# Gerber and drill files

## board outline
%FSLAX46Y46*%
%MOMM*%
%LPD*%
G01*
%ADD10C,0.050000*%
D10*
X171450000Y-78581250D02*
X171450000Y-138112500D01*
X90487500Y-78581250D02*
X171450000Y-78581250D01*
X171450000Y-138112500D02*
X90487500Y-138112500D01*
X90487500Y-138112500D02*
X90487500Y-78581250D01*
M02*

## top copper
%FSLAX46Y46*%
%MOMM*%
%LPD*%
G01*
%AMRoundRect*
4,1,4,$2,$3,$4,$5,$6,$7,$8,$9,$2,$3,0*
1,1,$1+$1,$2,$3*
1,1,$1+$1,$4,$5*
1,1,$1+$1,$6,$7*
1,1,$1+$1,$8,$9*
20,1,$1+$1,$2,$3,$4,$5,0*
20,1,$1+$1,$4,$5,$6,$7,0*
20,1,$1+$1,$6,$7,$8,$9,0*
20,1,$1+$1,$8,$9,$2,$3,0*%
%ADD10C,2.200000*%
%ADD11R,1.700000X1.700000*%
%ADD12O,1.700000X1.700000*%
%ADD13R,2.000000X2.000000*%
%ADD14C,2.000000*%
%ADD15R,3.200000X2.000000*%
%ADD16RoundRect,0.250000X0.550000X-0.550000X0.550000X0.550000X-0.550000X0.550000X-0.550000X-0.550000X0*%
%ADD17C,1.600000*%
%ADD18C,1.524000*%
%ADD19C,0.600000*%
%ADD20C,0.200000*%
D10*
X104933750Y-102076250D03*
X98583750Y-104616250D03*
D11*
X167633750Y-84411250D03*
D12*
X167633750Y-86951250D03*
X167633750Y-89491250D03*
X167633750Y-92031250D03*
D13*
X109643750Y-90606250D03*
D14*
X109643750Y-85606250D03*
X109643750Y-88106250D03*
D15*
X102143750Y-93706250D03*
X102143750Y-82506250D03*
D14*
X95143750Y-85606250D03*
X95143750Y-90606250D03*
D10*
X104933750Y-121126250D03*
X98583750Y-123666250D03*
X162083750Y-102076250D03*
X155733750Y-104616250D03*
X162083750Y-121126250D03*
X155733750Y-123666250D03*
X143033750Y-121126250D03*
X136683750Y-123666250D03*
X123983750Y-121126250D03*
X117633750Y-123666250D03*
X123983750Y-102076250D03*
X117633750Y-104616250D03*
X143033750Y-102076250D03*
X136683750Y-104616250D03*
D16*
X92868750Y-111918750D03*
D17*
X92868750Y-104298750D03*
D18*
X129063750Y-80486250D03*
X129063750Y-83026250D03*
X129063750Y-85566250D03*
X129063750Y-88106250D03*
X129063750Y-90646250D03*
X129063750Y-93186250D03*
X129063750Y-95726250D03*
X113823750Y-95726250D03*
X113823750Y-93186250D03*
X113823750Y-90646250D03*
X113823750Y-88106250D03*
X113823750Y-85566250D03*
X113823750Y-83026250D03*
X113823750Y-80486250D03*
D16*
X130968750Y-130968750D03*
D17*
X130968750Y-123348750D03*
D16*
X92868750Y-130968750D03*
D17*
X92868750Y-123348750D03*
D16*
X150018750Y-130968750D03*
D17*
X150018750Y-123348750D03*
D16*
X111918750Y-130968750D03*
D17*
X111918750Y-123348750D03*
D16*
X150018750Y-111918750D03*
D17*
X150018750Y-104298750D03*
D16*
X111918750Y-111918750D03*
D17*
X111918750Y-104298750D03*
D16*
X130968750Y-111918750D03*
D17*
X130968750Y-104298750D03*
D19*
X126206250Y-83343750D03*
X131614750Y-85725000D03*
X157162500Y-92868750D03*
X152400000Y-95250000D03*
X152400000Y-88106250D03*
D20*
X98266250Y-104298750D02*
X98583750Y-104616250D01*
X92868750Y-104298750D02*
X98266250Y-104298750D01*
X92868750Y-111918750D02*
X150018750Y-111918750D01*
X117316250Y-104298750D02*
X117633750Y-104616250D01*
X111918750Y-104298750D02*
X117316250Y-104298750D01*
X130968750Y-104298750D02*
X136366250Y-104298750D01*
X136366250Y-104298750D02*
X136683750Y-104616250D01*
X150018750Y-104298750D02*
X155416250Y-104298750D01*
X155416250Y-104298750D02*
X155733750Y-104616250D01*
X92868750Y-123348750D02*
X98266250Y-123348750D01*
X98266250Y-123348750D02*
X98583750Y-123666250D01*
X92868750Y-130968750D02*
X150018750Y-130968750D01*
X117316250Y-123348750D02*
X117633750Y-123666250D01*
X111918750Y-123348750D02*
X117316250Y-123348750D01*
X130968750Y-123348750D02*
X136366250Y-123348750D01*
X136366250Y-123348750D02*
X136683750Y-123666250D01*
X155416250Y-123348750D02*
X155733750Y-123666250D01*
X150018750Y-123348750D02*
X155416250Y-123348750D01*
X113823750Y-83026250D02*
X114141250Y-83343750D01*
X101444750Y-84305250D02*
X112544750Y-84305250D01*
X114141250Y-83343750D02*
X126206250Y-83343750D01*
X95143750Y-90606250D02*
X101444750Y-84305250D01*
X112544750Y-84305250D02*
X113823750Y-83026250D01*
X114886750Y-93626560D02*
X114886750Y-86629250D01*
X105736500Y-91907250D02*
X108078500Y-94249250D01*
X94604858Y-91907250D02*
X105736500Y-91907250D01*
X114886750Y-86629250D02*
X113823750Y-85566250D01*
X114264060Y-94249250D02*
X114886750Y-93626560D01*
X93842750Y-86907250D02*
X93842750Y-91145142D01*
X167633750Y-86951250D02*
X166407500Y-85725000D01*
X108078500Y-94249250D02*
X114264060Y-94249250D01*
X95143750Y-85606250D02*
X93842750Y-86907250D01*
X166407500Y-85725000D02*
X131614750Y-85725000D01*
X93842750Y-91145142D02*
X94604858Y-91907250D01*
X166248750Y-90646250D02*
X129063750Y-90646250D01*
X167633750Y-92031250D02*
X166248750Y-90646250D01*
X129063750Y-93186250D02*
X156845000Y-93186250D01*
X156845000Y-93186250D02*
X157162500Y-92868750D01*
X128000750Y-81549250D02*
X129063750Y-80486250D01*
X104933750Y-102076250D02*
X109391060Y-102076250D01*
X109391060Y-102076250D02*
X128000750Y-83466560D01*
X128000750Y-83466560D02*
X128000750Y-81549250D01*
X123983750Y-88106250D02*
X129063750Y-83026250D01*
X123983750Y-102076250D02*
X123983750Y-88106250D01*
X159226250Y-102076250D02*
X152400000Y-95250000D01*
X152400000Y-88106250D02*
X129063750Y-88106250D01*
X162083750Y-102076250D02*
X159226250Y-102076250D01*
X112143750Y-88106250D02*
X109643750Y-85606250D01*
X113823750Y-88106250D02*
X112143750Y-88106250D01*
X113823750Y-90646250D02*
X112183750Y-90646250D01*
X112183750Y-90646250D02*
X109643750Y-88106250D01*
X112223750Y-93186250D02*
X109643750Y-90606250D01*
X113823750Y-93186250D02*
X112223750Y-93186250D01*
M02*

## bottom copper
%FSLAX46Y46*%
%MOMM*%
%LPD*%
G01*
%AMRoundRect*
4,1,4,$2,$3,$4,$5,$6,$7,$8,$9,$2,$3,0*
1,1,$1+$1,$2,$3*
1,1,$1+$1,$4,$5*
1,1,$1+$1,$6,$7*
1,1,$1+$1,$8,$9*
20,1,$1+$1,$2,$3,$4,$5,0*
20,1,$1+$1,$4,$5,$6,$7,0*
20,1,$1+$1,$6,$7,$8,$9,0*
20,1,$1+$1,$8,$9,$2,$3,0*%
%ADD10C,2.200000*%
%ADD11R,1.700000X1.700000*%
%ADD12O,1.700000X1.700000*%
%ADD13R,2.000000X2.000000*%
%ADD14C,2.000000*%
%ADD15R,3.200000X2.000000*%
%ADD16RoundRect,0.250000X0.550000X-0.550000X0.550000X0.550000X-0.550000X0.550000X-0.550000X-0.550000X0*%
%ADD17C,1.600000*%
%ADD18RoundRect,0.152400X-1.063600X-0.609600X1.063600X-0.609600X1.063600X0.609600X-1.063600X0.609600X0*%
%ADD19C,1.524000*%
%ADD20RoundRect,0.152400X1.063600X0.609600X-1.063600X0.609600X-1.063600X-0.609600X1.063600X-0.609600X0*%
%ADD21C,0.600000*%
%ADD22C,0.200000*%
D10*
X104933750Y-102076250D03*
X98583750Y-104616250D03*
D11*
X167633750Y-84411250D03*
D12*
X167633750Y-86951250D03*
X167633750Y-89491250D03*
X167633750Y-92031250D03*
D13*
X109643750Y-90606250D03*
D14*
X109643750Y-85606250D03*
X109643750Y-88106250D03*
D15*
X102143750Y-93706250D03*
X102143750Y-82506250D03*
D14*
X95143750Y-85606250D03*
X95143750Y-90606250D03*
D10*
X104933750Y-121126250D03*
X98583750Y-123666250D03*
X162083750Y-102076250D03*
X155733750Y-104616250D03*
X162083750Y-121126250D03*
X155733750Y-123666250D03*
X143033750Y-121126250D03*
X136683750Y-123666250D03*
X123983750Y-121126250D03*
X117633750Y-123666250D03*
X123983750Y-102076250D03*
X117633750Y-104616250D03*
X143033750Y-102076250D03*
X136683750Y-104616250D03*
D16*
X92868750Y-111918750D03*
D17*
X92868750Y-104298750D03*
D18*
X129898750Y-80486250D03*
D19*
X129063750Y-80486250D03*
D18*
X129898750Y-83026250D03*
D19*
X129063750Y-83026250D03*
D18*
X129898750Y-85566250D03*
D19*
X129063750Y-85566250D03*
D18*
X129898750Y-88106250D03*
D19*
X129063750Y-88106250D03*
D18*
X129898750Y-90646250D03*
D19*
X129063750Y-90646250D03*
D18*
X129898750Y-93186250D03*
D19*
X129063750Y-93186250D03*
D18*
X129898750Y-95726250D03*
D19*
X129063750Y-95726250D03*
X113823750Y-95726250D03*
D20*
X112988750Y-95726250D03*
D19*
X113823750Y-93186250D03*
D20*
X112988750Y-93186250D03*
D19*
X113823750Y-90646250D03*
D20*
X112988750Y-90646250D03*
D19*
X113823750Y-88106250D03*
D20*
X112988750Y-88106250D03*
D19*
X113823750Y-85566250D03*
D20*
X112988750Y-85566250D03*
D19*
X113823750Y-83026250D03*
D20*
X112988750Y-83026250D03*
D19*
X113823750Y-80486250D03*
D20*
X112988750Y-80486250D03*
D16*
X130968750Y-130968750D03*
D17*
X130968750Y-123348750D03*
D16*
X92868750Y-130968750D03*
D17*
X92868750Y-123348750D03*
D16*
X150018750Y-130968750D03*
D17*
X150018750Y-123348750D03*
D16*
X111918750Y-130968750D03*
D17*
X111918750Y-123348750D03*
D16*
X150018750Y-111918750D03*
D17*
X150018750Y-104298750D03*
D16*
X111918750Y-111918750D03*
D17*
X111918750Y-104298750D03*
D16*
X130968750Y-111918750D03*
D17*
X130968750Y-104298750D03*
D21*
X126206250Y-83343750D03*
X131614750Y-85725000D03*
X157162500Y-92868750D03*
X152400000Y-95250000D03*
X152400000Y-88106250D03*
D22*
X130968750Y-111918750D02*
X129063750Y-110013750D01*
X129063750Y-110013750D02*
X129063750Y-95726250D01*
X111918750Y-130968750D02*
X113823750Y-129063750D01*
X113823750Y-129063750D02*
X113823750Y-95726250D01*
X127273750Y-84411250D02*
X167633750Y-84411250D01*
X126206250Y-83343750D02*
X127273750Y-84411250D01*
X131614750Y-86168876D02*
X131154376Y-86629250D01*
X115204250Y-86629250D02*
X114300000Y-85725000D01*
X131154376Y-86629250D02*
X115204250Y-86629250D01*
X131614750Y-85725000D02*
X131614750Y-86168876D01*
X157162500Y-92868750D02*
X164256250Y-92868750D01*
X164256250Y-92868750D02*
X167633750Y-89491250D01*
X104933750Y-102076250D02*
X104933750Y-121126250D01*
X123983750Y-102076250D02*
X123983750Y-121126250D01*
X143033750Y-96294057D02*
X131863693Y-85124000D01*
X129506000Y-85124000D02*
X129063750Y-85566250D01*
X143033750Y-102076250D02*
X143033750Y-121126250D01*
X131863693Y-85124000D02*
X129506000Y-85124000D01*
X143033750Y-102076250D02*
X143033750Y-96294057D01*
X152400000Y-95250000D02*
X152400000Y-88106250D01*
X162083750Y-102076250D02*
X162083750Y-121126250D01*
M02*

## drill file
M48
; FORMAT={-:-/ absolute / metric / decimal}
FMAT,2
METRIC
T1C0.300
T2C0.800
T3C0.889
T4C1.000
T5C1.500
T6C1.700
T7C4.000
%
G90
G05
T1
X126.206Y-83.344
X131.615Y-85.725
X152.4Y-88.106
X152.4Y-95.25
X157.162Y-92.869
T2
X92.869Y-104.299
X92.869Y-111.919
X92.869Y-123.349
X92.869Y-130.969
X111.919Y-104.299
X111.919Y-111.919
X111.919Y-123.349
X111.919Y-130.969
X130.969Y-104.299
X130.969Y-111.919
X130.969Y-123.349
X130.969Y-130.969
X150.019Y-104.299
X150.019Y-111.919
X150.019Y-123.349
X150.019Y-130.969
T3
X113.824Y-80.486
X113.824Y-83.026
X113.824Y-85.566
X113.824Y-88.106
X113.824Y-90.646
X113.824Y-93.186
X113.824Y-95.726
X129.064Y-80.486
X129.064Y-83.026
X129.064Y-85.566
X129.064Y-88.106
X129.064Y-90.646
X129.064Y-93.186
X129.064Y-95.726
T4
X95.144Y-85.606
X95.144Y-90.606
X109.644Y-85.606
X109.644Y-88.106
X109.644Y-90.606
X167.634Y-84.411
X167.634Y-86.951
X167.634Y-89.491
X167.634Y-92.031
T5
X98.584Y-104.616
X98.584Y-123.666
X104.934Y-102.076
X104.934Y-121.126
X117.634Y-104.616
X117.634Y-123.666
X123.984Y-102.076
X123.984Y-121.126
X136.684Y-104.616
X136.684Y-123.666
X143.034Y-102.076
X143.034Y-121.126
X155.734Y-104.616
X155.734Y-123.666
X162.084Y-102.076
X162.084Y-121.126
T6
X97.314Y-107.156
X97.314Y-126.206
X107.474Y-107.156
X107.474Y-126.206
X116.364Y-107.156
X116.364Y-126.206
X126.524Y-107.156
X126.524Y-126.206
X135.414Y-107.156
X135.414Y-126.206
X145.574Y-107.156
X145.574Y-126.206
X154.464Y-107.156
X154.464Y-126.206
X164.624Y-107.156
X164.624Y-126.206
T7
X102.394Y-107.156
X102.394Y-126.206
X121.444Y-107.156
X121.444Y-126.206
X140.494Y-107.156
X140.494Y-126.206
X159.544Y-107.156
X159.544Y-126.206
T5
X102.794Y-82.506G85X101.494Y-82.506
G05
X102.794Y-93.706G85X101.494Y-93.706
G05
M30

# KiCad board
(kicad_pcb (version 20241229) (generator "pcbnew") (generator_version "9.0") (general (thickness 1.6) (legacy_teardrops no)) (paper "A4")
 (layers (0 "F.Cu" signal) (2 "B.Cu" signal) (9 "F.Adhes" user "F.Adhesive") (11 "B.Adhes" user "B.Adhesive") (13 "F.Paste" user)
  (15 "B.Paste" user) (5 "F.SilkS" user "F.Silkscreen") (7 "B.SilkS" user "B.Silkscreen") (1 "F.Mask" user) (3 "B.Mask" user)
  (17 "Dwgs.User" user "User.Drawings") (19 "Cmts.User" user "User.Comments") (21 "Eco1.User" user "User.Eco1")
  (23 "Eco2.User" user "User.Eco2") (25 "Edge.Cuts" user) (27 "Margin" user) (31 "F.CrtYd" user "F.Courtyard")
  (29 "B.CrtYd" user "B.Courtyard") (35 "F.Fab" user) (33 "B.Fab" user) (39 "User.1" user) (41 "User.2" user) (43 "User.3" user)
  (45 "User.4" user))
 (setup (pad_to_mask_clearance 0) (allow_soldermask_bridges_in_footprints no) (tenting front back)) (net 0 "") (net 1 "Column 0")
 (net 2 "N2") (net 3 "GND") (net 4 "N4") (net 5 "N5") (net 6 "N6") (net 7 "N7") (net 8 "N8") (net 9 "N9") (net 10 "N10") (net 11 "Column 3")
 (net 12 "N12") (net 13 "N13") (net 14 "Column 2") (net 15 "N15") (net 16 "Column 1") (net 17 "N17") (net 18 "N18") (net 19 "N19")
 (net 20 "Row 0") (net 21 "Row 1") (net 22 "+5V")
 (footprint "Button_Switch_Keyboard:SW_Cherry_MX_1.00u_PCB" (layer "F.Cu") (at 104.93375 102.07625)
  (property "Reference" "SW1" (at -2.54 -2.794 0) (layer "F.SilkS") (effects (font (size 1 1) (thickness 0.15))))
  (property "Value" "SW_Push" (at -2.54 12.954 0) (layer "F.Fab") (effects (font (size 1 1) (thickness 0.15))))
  (pad "" np_thru_hole circle (at -7.62 5.08) (size 1.7 1.7) (drill 1.7) (layers "*.Cu" "*.Mask"))
  (pad "" np_thru_hole circle (at -2.54 5.08) (size 4 4) (drill 4) (layers "*.Cu" "*.Mask"))
  (pad "" np_thru_hole circle (at 2.54 5.08) (size 1.7 1.7) (drill 1.7) (layers "*.Cu" "*.Mask"))
  (pad "1" thru_hole circle (at 0 0) (size 2.2 2.2) (drill 1.5) (layers "*.Cu" "*.Mask") (remove_unused_layers no) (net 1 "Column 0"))
  (pad "2" thru_hole circle (at -6.35 2.54) (size 2.2 2.2) (drill 1.5) (layers "*.Cu" "*.Mask") (remove_unused_layers no) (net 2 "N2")))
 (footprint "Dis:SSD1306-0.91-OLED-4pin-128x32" (layer "F.Cu") (at 131.13375 82.22125)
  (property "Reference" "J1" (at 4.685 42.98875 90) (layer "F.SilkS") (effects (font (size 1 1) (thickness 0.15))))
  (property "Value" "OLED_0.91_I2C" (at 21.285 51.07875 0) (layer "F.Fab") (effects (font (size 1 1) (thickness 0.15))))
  (pad "1" thru_hole rect (at 36.5 2.19) (size 1.7 1.7) (drill 1) (layers "*.Cu" "*.Mask") (remove_unused_layers no) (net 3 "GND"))
  (pad "2" thru_hole oval (at 36.5 4.73) (size 1.7 1.7) (drill 1) (layers "*.Cu" "*.Mask") (remove_unused_layers no) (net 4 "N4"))
  (pad "3" thru_hole oval (at 36.5 7.27) (size 1.7 1.7) (drill 1) (layers "*.Cu" "*.Mask") (remove_unused_layers no) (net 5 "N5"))
  (pad "4" thru_hole oval (at 36.5 9.81) (size 1.7 1.7) (drill 1) (layers "*.Cu" "*.Mask") (remove_unused_layers no) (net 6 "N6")))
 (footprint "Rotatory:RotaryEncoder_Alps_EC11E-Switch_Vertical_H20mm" (layer "F.Cu") (at 109.64375 90.60625 180)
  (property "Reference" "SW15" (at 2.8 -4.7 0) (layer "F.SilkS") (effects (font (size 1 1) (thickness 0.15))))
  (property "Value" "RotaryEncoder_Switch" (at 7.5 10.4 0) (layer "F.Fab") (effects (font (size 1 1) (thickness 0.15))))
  (pad "A" thru_hole rect (at 0 0 180) (size 2 2) (drill 1) (layers "*.Cu" "*.Mask") (remove_unused_layers no) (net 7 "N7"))
  (pad "B" thru_hole circle (at 0 5 180) (size 2 2) (drill 1) (layers "*.Cu" "*.Mask") (remove_unused_layers no) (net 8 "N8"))
  (pad "C" thru_hole circle (at 0 2.5 180) (size 2 2) (drill 1) (layers "*.Cu" "*.Mask") (remove_unused_layers no) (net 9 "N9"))
  (pad "MP" thru_hole rect (at 7.5 -3.1 180) (size 3.2 2) (drill oval 2.8 1.5) (layers "*.Cu" "*.Mask") (remove_unused_layers no))
  (pad "MP" thru_hole rect (at 7.5 8.1 180) (size 3.2 2) (drill oval 2.8 1.5) (layers "*.Cu" "*.Mask") (remove_unused_layers no))
  (pad "S1" thru_hole circle (at 14.5 5 180) (size 2 2) (drill 1) (layers "*.Cu" "*.Mask") (remove_unused_layers no) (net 4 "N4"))
  (pad "S2" thru_hole circle (at 14.5 0 180) (size 2 2) (drill 1) (layers "*.Cu" "*.Mask") (remove_unused_layers no) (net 3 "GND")))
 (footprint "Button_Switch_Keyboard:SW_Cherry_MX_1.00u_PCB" (layer "F.Cu") (at 104.93375 121.12625)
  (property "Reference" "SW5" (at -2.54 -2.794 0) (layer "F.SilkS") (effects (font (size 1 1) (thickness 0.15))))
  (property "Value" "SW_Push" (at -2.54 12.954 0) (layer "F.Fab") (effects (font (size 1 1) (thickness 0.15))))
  (pad "" np_thru_hole circle (at -7.62 5.08) (size 1.7 1.7) (drill 1.7) (layers "*.Cu" "*.Mask"))
  (pad "" np_thru_hole circle (at -2.54 5.08) (size 4 4) (drill 4) (layers "*.Cu" "*.Mask"))
  (pad "" np_thru_hole circle (at 2.54 5.08) (size 1.7 1.7) (drill 1.7) (layers "*.Cu" "*.Mask"))
  (pad "1" thru_hole circle (at 0 0) (size 2.2 2.2) (drill 1.5) (layers "*.Cu" "*.Mask") (remove_unused_layers no) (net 1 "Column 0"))
  (pad "2" thru_hole circle (at -6.35 2.54) (size 2.2 2.2) (drill 1.5) (layers "*.Cu" "*.Mask") (remove_unused_layers no) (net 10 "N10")))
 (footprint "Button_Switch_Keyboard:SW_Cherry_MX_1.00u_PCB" (layer "F.Cu") (at 162.08375 102.07625)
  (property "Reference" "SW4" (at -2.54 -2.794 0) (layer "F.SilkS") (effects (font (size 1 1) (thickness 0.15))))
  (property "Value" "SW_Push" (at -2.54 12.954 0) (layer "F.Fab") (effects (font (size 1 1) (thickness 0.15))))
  (pad "" np_thru_hole circle (at -7.62 5.08) (size 1.7 1.7) (drill 1.7) (layers "*.Cu" "*.Mask"))
  (pad "" np_thru_hole circle (at -2.54 5.08) (size 4 4) (drill 4) (layers "*.Cu" "*.Mask"))
  (pad "" np_thru_hole circle (at 2.54 5.08) (size 1.7 1.7) (drill 1.7) (layers "*.Cu" "*.Mask"))
  (pad "1" thru_hole circle (at 0 0) (size 2.2 2.2) (drill 1.5) (layers "*.Cu" "*.Mask") (remove_unused_layers no) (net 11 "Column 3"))
  (pad "2" thru_hole circle (at -6.35 2.54) (size 2.2 2.2) (drill 1.5) (layers "*.Cu" "*.Mask") (remove_unused_layers no) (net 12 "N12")))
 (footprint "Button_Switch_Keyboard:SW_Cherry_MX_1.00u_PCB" (layer "F.Cu") (at 162.08375 121.12625)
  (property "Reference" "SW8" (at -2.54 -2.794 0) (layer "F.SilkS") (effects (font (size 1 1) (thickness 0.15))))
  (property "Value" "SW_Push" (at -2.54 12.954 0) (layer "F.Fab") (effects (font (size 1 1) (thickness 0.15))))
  (pad "" np_thru_hole circle (at -7.62 5.08) (size 1.7 1.7) (drill 1.7) (layers "*.Cu" "*.Mask"))
  (pad "" np_thru_hole circle (at -2.54 5.08) (size 4 4) (drill 4) (layers "*.Cu" "*.Mask"))
  (pad "" np_thru_hole circle (at 2.54 5.08) (size 1.7 1.7) (drill 1.7) (layers "*.Cu" "*.Mask"))
  (pad "1" thru_hole circle (at 0 0) (size 2.2 2.2) (drill 1.5) (layers "*.Cu" "*.Mask") (remove_unused_layers no) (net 11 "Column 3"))
  (pad "2" thru_hole circle (at -6.35 2.54) (size 2.2 2.2) (drill 1.5) (layers "*.Cu" "*.Mask") (remove_unused_layers no) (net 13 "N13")))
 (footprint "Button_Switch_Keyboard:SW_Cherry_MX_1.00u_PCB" (layer "F.Cu") (at 143.03375 121.12625)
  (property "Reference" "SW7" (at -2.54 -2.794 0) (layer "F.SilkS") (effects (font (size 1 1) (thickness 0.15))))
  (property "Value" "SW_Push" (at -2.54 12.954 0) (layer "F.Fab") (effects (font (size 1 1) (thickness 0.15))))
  (pad "" np_thru_hole circle (at -7.62 5.08) (size 1.7 1.7) (drill 1.7) (layers "*.Cu" "*.Mask"))
  (pad "" np_thru_hole circle (at -2.54 5.08) (size 4 4) (drill 4) (layers "*.Cu" "*.Mask"))
  (pad "" np_thru_hole circle (at 2.54 5.08) (size 1.7 1.7) (drill 1.7) (layers "*.Cu" "*.Mask"))
  (pad "1" thru_hole circle (at 0 0) (size 2.2 2.2) (drill 1.5) (layers "*.Cu" "*.Mask") (remove_unused_layers no) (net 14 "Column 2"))
  (pad "2" thru_hole circle (at -6.35 2.54) (size 2.2 2.2) (drill 1.5) (layers "*.Cu" "*.Mask") (remove_unused_layers no) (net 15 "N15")))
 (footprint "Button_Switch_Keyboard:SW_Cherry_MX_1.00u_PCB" (layer "F.Cu") (at 123.98375 121.12625)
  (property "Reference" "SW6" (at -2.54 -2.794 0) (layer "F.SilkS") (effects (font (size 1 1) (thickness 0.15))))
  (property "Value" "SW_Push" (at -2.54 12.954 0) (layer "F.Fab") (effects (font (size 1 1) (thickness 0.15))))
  (pad "" np_thru_hole circle (at -7.62 5.08) (size 1.7 1.7) (drill 1.7) (layers "*.Cu" "*.Mask"))
  (pad "" np_thru_hole circle (at -2.54 5.08) (size 4 4) (drill 4) (layers "*.Cu" "*.Mask"))
  (pad "" np_thru_hole circle (at 2.54 5.08) (size 1.7 1.7) (drill 1.7) (layers "*.Cu" "*.Mask"))
  (pad "1" thru_hole circle (at 0 0) (size 2.2 2.2) (drill 1.5) (layers "*.Cu" "*.Mask") (remove_unused_layers no) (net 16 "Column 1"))
  (pad "2" thru_hole circle (at -6.35 2.54) (size 2.2 2.2) (drill 1.5) (layers "*.Cu" "*.Mask") (remove_unused_layers no) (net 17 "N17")))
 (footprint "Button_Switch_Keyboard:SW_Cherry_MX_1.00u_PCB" (layer "F.Cu") (at 123.98375 102.07625)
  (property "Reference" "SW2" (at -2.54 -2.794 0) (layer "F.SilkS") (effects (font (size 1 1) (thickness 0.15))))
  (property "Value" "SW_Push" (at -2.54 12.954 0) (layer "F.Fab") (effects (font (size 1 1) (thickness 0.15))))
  (pad "" np_thru_hole circle (at -7.62 5.08) (size 1.7 1.7) (drill 1.7) (layers "*.Cu" "*.Mask"))
  (pad "" np_thru_hole circle (at -2.54 5.08) (size 4 4) (drill 4) (layers "*.Cu" "*.Mask"))
  (pad "" np_thru_hole circle (at 2.54 5.08) (size 1.7 1.7) (drill 1.7) (layers "*.Cu" "*.Mask"))
  (pad "1" thru_hole circle (at 0 0) (size 2.2 2.2) (drill 1.5) (layers "*.Cu" "*.Mask") (remove_unused_layers no) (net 16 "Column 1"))
  (pad "2" thru_hole circle (at -6.35 2.54) (size 2.2 2.2) (drill 1.5) (layers "*.Cu" "*.Mask") (remove_unused_layers no) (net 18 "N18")))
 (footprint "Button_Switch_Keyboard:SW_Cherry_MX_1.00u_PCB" (layer "F.Cu") (at 143.03375 102.07625)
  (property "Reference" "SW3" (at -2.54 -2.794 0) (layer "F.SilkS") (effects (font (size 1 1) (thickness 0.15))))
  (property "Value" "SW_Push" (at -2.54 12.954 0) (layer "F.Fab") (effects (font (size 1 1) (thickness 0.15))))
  (pad "" np_thru_hole circle (at -7.62 5.08) (size 1.7 1.7) (drill 1.7) (layers "*.Cu" "*.Mask"))
  (pad "" np_thru_hole circle (at -2.54 5.08) (size 4 4) (drill 4) (layers "*.Cu" "*.Mask"))
  (pad "" np_thru_hole circle (at 2.54 5.08) (size 1.7 1.7) (drill 1.7) (layers "*.Cu" "*.Mask"))
  (pad "1" thru_hole circle (at 0 0) (size 2.2 2.2) (drill 1.5) (layers "*.Cu" "*.Mask") (remove_unused_layers no) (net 14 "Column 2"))
  (pad "2" thru_hole circle (at -6.35 2.54) (size 2.2 2.2) (drill 1.5) (layers "*.Cu" "*.Mask") (remove_unused_layers no) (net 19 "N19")))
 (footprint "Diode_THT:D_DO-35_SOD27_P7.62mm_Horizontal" (layer "B.Cu") (at 92.86875 111.91875 90)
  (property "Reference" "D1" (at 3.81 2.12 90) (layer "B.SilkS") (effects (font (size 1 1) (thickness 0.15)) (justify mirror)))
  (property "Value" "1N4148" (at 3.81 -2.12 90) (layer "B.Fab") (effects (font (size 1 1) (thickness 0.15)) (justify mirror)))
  (pad "1" thru_hole roundrect (at 0 0 90) (size 1.6 1.6) (drill 0.8) (layers "*.Cu" "*.Mask") (remove_unused_layers no)
   (roundrect_rratio 0.15625) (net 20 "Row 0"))
  (pad "2" thru_hole circle (at 7.62 0 90) (size 1.6 1.6) (drill 0.8) (layers "*.Cu" "*.Mask") (remove_unused_layers no) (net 2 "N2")))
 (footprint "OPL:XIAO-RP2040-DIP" (layer "B.Cu") (at 121.44375 88.10625 180)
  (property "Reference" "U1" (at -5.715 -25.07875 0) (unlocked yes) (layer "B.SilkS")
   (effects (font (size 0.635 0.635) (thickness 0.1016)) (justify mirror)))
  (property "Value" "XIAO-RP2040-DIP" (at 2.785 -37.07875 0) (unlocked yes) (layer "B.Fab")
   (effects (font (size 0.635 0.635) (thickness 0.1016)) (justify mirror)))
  (pad "1" smd roundrect (at -8.455 7.62) (size 2.432 1.524) (layers "B.Cu" "B.Mask") (roundrect_rratio 0.1) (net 1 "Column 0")
   (thermal_bridge_angle 45))
  (pad "1" thru_hole circle (at -7.62 7.62) (size 1.524 1.524) (drill 0.889) (layers "*.Cu" "*.Mask") (remove_unused_layers no)
   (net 1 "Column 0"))
  (pad "2" smd roundrect (at -8.455 5.08) (size 2.432 1.524) (layers "B.Cu" "B.Mask") (roundrect_rratio 0.1) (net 16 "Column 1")
   (thermal_bridge_angle 45))
  (pad "2" thru_hole circle (at -7.62 5.08) (size 1.524 1.524) (drill 0.889) (layers "*.Cu" "*.Mask") (remove_unused_layers no)
   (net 16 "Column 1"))
  (pad "3" smd roundrect (at -8.455 2.54) (size 2.432 1.524) (layers "B.Cu" "B.Mask") (roundrect_rratio 0.1) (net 14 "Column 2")
   (thermal_bridge_angle 45))
  (pad "3" thru_hole circle (at -7.62 2.54) (size 1.524 1.524) (drill 0.889) (layers "*.Cu" "*.Mask") (remove_unused_layers no)
   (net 14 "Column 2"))
  (pad "4" smd roundrect (at -8.455 0) (size 2.432 1.524) (layers "B.Cu" "B.Mask") (roundrect_rratio 0.1) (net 11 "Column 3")
   (thermal_bridge_angle 45))
  (pad "4" thru_hole circle (at -7.62 0) (size 1.524 1.524) (drill 0.889) (layers "*.Cu" "*.Mask") (remove_unused_layers no)
   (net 11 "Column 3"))
  (pad "5" smd roundrect (at -8.455 -2.54) (size 2.432 1.524) (layers "B.Cu" "B.Mask") (roundrect_rratio 0.1) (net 6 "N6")
   (thermal_bridge_angle 45))
  (pad "5" thru_hole circle (at -7.62 -2.54) (size 1.524 1.524) (drill 0.889) (layers "*.Cu" "*.Mask") (remove_unused_layers no)
   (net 6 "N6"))
  (pad "6" smd roundrect (at -8.455 -5.08) (size 2.432 1.524) (layers "B.Cu" "B.Mask") (roundrect_rratio 0.1) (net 5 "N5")
   (thermal_bridge_angle 45))
  (pad "6" thru_hole circle (at -7.62 -5.08) (size 1.524 1.524) (drill 0.889) (layers "*.Cu" "*.Mask") (remove_unused_layers no)
   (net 5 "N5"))
  (pad "7" smd roundrect (at -8.455 -7.62) (size 2.432 1.524) (layers "B.Cu" "B.Mask") (roundrect_rratio 0.1) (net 20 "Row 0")
   (thermal_bridge_angle 45))
  (pad "7" thru_hole circle (at -7.62 -7.62) (size 1.524 1.524) (drill 0.889) (layers "*.Cu" "*.Mask") (remove_unused_layers no)
   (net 20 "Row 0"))
  (pad "8" thru_hole circle (at 7.62 -7.62 180) (size 1.524 1.524) (drill 0.889) (layers "*.Cu" "*.Mask") (remove_unused_layers no)
   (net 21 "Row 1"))
  (pad "8" smd roundrect (at 8.455 -7.62 180) (size 2.432 1.524) (layers "B.Cu" "B.Mask") (roundrect_rratio 0.1) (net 21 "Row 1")
   (thermal_bridge_angle 45))
  (pad "9" thru_hole circle (at 7.62 -5.08 180) (size 1.524 1.524) (drill 0.889) (layers "*.Cu" "*.Mask") (remove_unused_layers no)
   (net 7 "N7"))
  (pad "9" smd roundrect (at 8.455 -5.08 180) (size 2.432 1.524) (layers "B.Cu" "B.Mask") (roundrect_rratio 0.1) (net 7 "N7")
   (thermal_bridge_angle 45))
  (pad "10" thru_hole circle (at 7.62 -2.54 180) (size 1.524 1.524) (drill 0.889) (layers "*.Cu" "*.Mask") (remove_unused_layers no)
   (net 9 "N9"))
  (pad "10" smd roundrect (at 8.455 -2.54 180) (size 2.432 1.524) (layers "B.Cu" "B.Mask") (roundrect_rratio 0.1) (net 9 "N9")
   (thermal_bridge_angle 45))
  (pad "11" thru_hole circle (at 7.62 0 180) (size 1.524 1.524) (drill 0.889) (layers "*.Cu" "*.Mask") (remove_unused_layers no)
   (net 8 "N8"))
  (pad "11" smd roundrect (at 8.455 0 180) (size 2.432 1.524) (layers "B.Cu" "B.Mask") (roundrect_rratio 0.1) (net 8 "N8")
   (thermal_bridge_angle 45))
  (pad "12" thru_hole circle (at 7.62 2.54 180) (size 1.524 1.524) (drill 0.889) (layers "*.Cu" "*.Mask") (remove_unused_layers no)
   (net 4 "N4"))
  (pad "12" smd roundrect (at 8.455 2.54 180) (size 2.432 1.524) (layers "B.Cu" "B.Mask") (roundrect_rratio 0.1) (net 4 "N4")
   (thermal_bridge_angle 45))
  (pad "13" thru_hole circle (at 7.62 5.08 180) (size 1.524 1.524) (drill 0.889) (layers "*.Cu" "*.Mask") (remove_unused_layers no)
   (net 3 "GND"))
  (pad "13" smd roundrect (at 8.455 5.08 180) (size 2.432 1.524) (layers "B.Cu" "B.Mask") (roundrect_rratio 0.1) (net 3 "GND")
   (thermal_bridge_angle 45))
  (pad "14" thru_hole circle (at 7.62 7.62 180) (size 1.524 1.524) (drill 0.889) (layers "*.Cu" "*.Mask") (remove_unused_layers no)
   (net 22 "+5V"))
  (pad "14" smd roundrect (at 8.455 7.62 180) (size 2.432 1.524) (layers "B.Cu" "B.Mask") (roundrect_rratio 0.1) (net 22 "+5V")
   (thermal_bridge_angle 45)))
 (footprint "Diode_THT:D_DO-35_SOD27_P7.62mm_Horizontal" (layer "B.Cu") (at 130.96875 130.96875 90)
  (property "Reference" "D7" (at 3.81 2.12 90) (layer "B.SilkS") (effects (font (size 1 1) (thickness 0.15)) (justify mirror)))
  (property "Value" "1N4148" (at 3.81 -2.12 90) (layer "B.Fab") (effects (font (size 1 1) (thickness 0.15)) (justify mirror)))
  (pad "1" thru_hole roundrect (at 0 0 90) (size 1.6 1.6) (drill 0.8) (layers "*.Cu" "*.Mask") (remove_unused_layers no)
   (roundrect_rratio 0.15625) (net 21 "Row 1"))
  (pad "2" thru_hole circle (at 7.62 0 90) (size 1.6 1.6) (drill 0.8) (layers "*.Cu" "*.Mask") (remove_unused_layers no) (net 15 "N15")))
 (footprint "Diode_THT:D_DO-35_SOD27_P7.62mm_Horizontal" (layer "B.Cu") (at 92.86875 130.96875 90)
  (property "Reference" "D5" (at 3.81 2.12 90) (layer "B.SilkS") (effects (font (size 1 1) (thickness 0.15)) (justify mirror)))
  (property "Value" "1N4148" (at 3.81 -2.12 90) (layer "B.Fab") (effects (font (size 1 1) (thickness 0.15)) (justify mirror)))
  (pad "1" thru_hole roundrect (at 0 0 90) (size 1.6 1.6) (drill 0.8) (layers "*.Cu" "*.Mask") (remove_unused_layers no)
   (roundrect_rratio 0.15625) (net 21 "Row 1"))
  (pad "2" thru_hole circle (at 7.62 0 90) (size 1.6 1.6) (drill 0.8) (layers "*.Cu" "*.Mask") (remove_unused_layers no) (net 10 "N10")))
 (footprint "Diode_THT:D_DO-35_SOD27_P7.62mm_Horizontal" (layer "B.Cu") (at 150.01875 130.96875 90)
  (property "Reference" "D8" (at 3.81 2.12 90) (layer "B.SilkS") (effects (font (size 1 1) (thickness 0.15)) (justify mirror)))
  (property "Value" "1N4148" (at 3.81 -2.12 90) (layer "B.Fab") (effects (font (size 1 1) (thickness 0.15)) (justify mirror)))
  (pad "1" thru_hole roundrect (at 0 0 90) (size 1.6 1.6) (drill 0.8) (layers "*.Cu" "*.Mask") (remove_unused_layers no)
   (roundrect_rratio 0.15625) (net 21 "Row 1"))
  (pad "2" thru_hole circle (at 7.62 0 90) (size 1.6 1.6) (drill 0.8) (layers "*.Cu" "*.Mask") (remove_unused_layers no) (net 13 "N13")))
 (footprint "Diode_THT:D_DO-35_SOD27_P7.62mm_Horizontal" (layer "B.Cu") (at 111.91875 130.96875 90)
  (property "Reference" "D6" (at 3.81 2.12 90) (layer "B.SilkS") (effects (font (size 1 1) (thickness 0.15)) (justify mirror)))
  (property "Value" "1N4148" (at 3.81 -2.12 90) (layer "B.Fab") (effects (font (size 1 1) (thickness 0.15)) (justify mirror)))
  (pad "1" thru_hole roundrect (at 0 0 90) (size 1.6 1.6) (drill 0.8) (layers "*.Cu" "*.Mask") (remove_unused_layers no)
   (roundrect_rratio 0.15625) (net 21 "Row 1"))
  (pad "2" thru_hole circle (at 7.62 0 90) (size 1.6 1.6) (drill 0.8) (layers "*.Cu" "*.Mask") (remove_unused_layers no) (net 17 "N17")))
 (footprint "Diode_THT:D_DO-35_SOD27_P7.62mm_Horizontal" (layer "B.Cu") (at 150.01875 111.91875 90)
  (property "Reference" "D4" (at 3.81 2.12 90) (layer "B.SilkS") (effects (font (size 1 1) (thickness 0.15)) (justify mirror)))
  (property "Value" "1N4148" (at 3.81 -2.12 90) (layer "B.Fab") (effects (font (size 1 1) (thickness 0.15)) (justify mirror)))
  (pad "1" thru_hole roundrect (at 0 0 90) (size 1.6 1.6) (drill 0.8) (layers "*.Cu" "*.Mask") (remove_unused_layers no)
   (roundrect_rratio 0.15625) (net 20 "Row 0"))
  (pad "2" thru_hole circle (at 7.62 0 90) (size 1.6 1.6) (drill 0.8) (layers "*.Cu" "*.Mask") (remove_unused_layers no) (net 12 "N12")))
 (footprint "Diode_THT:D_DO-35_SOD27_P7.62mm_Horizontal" (layer "B.Cu") (at 111.91875 111.91875 90)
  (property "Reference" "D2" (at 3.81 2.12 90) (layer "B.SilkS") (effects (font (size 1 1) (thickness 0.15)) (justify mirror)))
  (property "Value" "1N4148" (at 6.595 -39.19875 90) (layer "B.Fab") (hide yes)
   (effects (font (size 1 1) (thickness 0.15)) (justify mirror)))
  (pad "1" thru_hole roundrect (at 0 0 90) (size 1.6 1.6) (drill 0.8) (layers "*.Cu" "*.Mask") (remove_unused_layers no)
   (roundrect_rratio 0.15625) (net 20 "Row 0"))
  (pad "2" thru_hole circle (at 7.62 0 90) (size 1.6 1.6) (drill 0.8) (layers "*.Cu" "*.Mask") (remove_unused_layers no) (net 18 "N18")))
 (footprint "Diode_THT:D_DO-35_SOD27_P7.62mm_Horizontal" (layer "B.Cu") (at 130.96875 111.91875 90)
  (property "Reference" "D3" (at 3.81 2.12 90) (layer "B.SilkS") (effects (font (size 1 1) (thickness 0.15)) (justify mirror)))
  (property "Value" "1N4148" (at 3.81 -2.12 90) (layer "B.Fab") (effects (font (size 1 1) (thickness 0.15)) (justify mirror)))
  (pad "1" thru_hole roundrect (at 0 0 90) (size 1.6 1.6) (drill 0.8) (layers "*.Cu" "*.Mask") (remove_unused_layers no)
   (roundrect_rratio 0.15625) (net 20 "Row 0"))
  (pad "2" thru_hole circle (at 7.62 0 90) (size 1.6 1.6) (drill 0.8) (layers "*.Cu" "*.Mask") (remove_unused_layers no) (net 19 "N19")))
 (gr_line (start 171.45 78.58125) (end 171.45 138.1125) (stroke (width 0.05) (type default)) (layer "Edge.Cuts"))
 (gr_line (start 90.4875 78.58125) (end 171.45 78.58125) (stroke (width 0.05) (type default)) (layer "Edge.Cuts"))
 (gr_line (start 171.45 138.1125) (end 90.4875 138.1125) (stroke (width 0.05) (type default)) (layer "Edge.Cuts"))
 (gr_line (start 90.4875 138.1125) (end 90.4875 78.58125) (stroke (width 0.05) (type default)) (layer "Edge.Cuts"))
 (segment (start 98.26625 104.29875) (end 98.58375 104.61625) (width 0.2) (layer "F.Cu") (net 2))
 (segment (start 92.86875 104.29875) (end 98.26625 104.29875) (width 0.2) (layer "F.Cu") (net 2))
 (segment (start 92.86875 111.91875) (end 150.01875 111.91875) (width 0.2) (layer "F.Cu") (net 20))
 (segment (start 130.96875 111.91875) (end 129.06375 110.01375) (width 0.2) (layer "B.Cu") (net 20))
 (segment (start 129.06375 110.01375) (end 129.06375 95.72625) (width 0.2) (layer "B.Cu") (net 20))
 (segment (start 117.31625 104.29875) (end 117.63375 104.61625) (width 0.2) (layer "F.Cu") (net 18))
 (segment (start 111.91875 104.29875) (end 117.31625 104.29875) (width 0.2) (layer "F.Cu") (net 18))
 (segment (start 130.96875 104.29875) (end 136.36625 104.29875) (width 0.2) (layer "F.Cu") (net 19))
 (segment (start 136.36625 104.29875) (end 136.68375 104.61625) (width 0.2) (layer "F.Cu") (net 19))
 (segment (start 150.01875 104.29875) (end 155.41625 104.29875) (width 0.2) (layer "F.Cu") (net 12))
 (segment (start 155.41625 104.29875) (end 155.73375 104.61625) (width 0.2) (layer "F.Cu") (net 12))
 (segment (start 92.86875 123.34875) (end 98.26625 123.34875) (width 0.2) (layer "F.Cu") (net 10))
 (segment (start 98.26625 123.34875) (end 98.58375 123.66625) (width 0.2) (layer "F.Cu") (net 10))
 (segment (start 92.86875 130.96875) (end 150.01875 130.96875) (width 0.2) (layer "F.Cu") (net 21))
 (segment (start 111.91875 130.96875) (end 113.82375 129.06375) (width 0.2) (layer "B.Cu") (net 21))
 (segment (start 113.82375 129.06375) (end 113.82375 95.72625) (width 0.2) (layer "B.Cu") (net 21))
 (segment (start 117.31625 123.34875) (end 117.63375 123.66625) (width 0.2) (layer "F.Cu") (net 17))
 (segment (start 111.91875 123.34875) (end 117.31625 123.34875) (width 0.2) (layer "F.Cu") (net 17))
 (segment (start 130.96875 123.34875) (end 136.36625 123.34875) (width 0.2) (layer "F.Cu") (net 15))
 (segment (start 136.36625 123.34875) (end 136.68375 123.66625) (width 0.2) (layer "F.Cu") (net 15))
 (segment (start 155.41625 123.34875) (end 155.73375 123.66625) (width 0.2) (layer "F.Cu") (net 13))
 (segment (start 150.01875 123.34875) (end 155.41625 123.34875) (width 0.2) (layer "F.Cu") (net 13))
 (segment (start 113.82375 83.02625) (end 114.14125 83.34375) (width 0.2) (layer "F.Cu") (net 3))
 (segment (start 101.44475 84.30525) (end 112.54475 84.30525) (width 0.2) (layer "F.Cu") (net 3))
 (segment (start 114.14125 83.34375) (end 126.20625 83.34375) (width 0.2) (layer "F.Cu") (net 3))
 (segment (start 95.14375 90.60625) (end 101.44475 84.30525) (width 0.2) (layer "F.Cu") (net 3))
 (segment (start 112.54475 84.30525) (end 113.82375 83.02625) (width 0.2) (layer "F.Cu") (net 3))
 (via (at 126.20625 83.34375) (size 0.6) (drill 0.3) (layers "F.Cu" "B.Cu") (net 3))
 (segment (start 127.27375 84.41125) (end 167.63375 84.41125) (width 0.2) (layer "B.Cu") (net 3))
 (segment (start 126.20625 83.34375) (end 127.27375 84.41125) (width 0.2) (layer "B.Cu") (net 3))
 (segment (start 114.88675 93.62656) (end 114.88675 86.62925) (width 0.2) (layer "F.Cu") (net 4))
 (segment (start 105.7365 91.90725) (end 108.0785 94.24925) (width 0.2) (layer "F.Cu") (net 4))
 (segment (start 94.604858 91.90725) (end 105.7365 91.90725) (width 0.2) (layer "F.Cu") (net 4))
 (segment (start 114.88675 86.62925) (end 113.82375 85.56625) (width 0.2) (layer "F.Cu") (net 4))
 (segment (start 114.26406 94.24925) (end 114.88675 93.62656) (width 0.2) (layer "F.Cu") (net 4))
 (segment (start 93.84275 86.90725) (end 93.84275 91.145142) (width 0.2) (layer "F.Cu") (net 4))
 (segment (start 167.63375 86.95125) (end 166.4075 85.725) (width 0.2) (layer "F.Cu") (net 4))
 (segment (start 108.0785 94.24925) (end 114.26406 94.24925) (width 0.2) (layer "F.Cu") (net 4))
 (segment (start 95.14375 85.60625) (end 93.84275 86.90725) (width 0.2) (layer "F.Cu") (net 4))
 (segment (start 166.4075 85.725) (end 131.61475 85.725) (width 0.2) (layer "F.Cu") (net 4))
 (segment (start 93.84275 91.145142) (end 94.604858 91.90725) (width 0.2) (layer "F.Cu") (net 4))
 (via (at 131.61475 85.725) (size 0.6) (drill 0.3) (layers "F.Cu" "B.Cu") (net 4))
 (segment (start 131.61475 86.168876) (end 131.154376 86.62925) (width 0.2) (layer "B.Cu") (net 4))
 (segment (start 115.20425 86.62925) (end 114.3 85.725) (width 0.2) (layer "B.Cu") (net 4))
 (segment (start 131.154376 86.62925) (end 115.20425 86.62925) (width 0.2) (layer "B.Cu") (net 4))
 (segment (start 131.61475 85.725) (end 131.61475 86.168876) (width 0.2) (layer "B.Cu") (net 4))
 (segment (start 166.24875 90.64625) (end 129.06375 90.64625) (width 0.2) (layer "F.Cu") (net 6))
 (segment (start 167.63375 92.03125) (end 166.24875 90.64625) (width 0.2) (layer "F.Cu") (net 6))
 (segment (start 129.06375 93.18625) (end 156.845 93.18625) (width 0.2) (layer "F.Cu") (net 5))
 (segment (start 156.845 93.18625) (end 157.1625 92.86875) (width 0.2) (layer "F.Cu") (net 5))
 (via (at 157.1625 92.86875) (size 0.6) (drill 0.3) (layers "F.Cu" "B.Cu") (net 5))
 (segment (start 157.1625 92.86875) (end 164.25625 92.86875) (width 0.2) (layer "B.Cu") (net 5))
 (segment (start 164.25625 92.86875) (end 167.63375 89.49125) (width 0.2) (layer "B.Cu") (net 5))
 (segment (start 128.00075 81.54925) (end 129.06375 80.48625) (width 0.2) (layer "F.Cu") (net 1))
 (segment (start 104.93375 102.07625) (end 109.39106 102.07625) (width 0.2) (layer "F.Cu") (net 1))
 (segment (start 109.39106 102.07625) (end 128.00075 83.46656) (width 0.2) (layer "F.Cu") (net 1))
 (segment (start 128.00075 83.46656) (end 128.00075 81.54925) (width 0.2) (layer "F.Cu") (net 1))
 (segment (start 104.93375 102.07625) (end 104.93375 121.12625) (width 0.2) (layer "B.Cu") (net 1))
 (segment (start 123.98375 88.10625) (end 129.06375 83.02625) (width 0.2) (layer "F.Cu") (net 16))
 (segment (start 123.98375 102.07625) (end 123.98375 88.10625) (width 0.2) (layer "F.Cu") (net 16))
 (segment (start 123.98375 102.07625) (end 123.98375 121.12625) (width 0.2) (layer "B.Cu") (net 16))
 (segment (start 143.03375 96.294057) (end 131.863693 85.124) (width 0.2) (layer "B.Cu") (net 14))
 (segment (start 129.506 85.124) (end 129.06375 85.56625) (width 0.2) (layer "B.Cu") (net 14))
 (segment (start 143.03375 102.07625) (end 143.03375 121.12625) (width 0.2) (layer "B.Cu") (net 14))
 (segment (start 131.863693 85.124) (end 129.506 85.124) (width 0.2) (layer "B.Cu") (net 14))
 (segment (start 143.03375 102.07625) (end 143.03375 96.294057) (width 0.2) (layer "B.Cu") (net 14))
 (segment (start 159.22625 102.07625) (end 152.4 95.25) (width 0.2) (layer "F.Cu") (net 11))
 (segment (start 152.4 88.10625) (end 129.06375 88.10625) (width 0.2) (layer "F.Cu") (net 11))
 (segment (start 162.08375 102.07625) (end 159.22625 102.07625) (width 0.2) (layer "F.Cu") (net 11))
 (via (at 152.4 95.25) (size 0.6) (drill 0.3) (layers "F.Cu" "B.Cu") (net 11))
 (via (at 152.4 88.10625) (size 0.6) (drill 0.3) (layers "F.Cu" "B.Cu") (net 11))
 (segment (start 152.4 95.25) (end 152.4 88.10625) (width 0.2) (layer "B.Cu") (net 11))
 (segment (start 162.08375 102.07625) (end 162.08375 121.12625) (width 0.2) (layer "B.Cu") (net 11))
 (segment (start 112.14375 88.10625) (end 109.64375 85.60625) (width 0.2) (layer "F.Cu") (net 8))
 (segment (start 113.82375 88.10625) (end 112.14375 88.10625) (width 0.2) (layer "F.Cu") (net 8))
 (segment (start 113.82375 90.64625) (end 112.18375 90.64625) (width 0.2) (layer "F.Cu") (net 9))
 (segment (start 112.18375 90.64625) (end 109.64375 88.10625) (width 0.2) (layer "F.Cu") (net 9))
 (segment (start 112.22375 93.18625) (end 109.64375 90.60625) (width 0.2) (layer "F.Cu") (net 7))
 (segment (start 113.82375 93.18625) (end 112.22375 93.18625) (width 0.2) (layer "F.Cu") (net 7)))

